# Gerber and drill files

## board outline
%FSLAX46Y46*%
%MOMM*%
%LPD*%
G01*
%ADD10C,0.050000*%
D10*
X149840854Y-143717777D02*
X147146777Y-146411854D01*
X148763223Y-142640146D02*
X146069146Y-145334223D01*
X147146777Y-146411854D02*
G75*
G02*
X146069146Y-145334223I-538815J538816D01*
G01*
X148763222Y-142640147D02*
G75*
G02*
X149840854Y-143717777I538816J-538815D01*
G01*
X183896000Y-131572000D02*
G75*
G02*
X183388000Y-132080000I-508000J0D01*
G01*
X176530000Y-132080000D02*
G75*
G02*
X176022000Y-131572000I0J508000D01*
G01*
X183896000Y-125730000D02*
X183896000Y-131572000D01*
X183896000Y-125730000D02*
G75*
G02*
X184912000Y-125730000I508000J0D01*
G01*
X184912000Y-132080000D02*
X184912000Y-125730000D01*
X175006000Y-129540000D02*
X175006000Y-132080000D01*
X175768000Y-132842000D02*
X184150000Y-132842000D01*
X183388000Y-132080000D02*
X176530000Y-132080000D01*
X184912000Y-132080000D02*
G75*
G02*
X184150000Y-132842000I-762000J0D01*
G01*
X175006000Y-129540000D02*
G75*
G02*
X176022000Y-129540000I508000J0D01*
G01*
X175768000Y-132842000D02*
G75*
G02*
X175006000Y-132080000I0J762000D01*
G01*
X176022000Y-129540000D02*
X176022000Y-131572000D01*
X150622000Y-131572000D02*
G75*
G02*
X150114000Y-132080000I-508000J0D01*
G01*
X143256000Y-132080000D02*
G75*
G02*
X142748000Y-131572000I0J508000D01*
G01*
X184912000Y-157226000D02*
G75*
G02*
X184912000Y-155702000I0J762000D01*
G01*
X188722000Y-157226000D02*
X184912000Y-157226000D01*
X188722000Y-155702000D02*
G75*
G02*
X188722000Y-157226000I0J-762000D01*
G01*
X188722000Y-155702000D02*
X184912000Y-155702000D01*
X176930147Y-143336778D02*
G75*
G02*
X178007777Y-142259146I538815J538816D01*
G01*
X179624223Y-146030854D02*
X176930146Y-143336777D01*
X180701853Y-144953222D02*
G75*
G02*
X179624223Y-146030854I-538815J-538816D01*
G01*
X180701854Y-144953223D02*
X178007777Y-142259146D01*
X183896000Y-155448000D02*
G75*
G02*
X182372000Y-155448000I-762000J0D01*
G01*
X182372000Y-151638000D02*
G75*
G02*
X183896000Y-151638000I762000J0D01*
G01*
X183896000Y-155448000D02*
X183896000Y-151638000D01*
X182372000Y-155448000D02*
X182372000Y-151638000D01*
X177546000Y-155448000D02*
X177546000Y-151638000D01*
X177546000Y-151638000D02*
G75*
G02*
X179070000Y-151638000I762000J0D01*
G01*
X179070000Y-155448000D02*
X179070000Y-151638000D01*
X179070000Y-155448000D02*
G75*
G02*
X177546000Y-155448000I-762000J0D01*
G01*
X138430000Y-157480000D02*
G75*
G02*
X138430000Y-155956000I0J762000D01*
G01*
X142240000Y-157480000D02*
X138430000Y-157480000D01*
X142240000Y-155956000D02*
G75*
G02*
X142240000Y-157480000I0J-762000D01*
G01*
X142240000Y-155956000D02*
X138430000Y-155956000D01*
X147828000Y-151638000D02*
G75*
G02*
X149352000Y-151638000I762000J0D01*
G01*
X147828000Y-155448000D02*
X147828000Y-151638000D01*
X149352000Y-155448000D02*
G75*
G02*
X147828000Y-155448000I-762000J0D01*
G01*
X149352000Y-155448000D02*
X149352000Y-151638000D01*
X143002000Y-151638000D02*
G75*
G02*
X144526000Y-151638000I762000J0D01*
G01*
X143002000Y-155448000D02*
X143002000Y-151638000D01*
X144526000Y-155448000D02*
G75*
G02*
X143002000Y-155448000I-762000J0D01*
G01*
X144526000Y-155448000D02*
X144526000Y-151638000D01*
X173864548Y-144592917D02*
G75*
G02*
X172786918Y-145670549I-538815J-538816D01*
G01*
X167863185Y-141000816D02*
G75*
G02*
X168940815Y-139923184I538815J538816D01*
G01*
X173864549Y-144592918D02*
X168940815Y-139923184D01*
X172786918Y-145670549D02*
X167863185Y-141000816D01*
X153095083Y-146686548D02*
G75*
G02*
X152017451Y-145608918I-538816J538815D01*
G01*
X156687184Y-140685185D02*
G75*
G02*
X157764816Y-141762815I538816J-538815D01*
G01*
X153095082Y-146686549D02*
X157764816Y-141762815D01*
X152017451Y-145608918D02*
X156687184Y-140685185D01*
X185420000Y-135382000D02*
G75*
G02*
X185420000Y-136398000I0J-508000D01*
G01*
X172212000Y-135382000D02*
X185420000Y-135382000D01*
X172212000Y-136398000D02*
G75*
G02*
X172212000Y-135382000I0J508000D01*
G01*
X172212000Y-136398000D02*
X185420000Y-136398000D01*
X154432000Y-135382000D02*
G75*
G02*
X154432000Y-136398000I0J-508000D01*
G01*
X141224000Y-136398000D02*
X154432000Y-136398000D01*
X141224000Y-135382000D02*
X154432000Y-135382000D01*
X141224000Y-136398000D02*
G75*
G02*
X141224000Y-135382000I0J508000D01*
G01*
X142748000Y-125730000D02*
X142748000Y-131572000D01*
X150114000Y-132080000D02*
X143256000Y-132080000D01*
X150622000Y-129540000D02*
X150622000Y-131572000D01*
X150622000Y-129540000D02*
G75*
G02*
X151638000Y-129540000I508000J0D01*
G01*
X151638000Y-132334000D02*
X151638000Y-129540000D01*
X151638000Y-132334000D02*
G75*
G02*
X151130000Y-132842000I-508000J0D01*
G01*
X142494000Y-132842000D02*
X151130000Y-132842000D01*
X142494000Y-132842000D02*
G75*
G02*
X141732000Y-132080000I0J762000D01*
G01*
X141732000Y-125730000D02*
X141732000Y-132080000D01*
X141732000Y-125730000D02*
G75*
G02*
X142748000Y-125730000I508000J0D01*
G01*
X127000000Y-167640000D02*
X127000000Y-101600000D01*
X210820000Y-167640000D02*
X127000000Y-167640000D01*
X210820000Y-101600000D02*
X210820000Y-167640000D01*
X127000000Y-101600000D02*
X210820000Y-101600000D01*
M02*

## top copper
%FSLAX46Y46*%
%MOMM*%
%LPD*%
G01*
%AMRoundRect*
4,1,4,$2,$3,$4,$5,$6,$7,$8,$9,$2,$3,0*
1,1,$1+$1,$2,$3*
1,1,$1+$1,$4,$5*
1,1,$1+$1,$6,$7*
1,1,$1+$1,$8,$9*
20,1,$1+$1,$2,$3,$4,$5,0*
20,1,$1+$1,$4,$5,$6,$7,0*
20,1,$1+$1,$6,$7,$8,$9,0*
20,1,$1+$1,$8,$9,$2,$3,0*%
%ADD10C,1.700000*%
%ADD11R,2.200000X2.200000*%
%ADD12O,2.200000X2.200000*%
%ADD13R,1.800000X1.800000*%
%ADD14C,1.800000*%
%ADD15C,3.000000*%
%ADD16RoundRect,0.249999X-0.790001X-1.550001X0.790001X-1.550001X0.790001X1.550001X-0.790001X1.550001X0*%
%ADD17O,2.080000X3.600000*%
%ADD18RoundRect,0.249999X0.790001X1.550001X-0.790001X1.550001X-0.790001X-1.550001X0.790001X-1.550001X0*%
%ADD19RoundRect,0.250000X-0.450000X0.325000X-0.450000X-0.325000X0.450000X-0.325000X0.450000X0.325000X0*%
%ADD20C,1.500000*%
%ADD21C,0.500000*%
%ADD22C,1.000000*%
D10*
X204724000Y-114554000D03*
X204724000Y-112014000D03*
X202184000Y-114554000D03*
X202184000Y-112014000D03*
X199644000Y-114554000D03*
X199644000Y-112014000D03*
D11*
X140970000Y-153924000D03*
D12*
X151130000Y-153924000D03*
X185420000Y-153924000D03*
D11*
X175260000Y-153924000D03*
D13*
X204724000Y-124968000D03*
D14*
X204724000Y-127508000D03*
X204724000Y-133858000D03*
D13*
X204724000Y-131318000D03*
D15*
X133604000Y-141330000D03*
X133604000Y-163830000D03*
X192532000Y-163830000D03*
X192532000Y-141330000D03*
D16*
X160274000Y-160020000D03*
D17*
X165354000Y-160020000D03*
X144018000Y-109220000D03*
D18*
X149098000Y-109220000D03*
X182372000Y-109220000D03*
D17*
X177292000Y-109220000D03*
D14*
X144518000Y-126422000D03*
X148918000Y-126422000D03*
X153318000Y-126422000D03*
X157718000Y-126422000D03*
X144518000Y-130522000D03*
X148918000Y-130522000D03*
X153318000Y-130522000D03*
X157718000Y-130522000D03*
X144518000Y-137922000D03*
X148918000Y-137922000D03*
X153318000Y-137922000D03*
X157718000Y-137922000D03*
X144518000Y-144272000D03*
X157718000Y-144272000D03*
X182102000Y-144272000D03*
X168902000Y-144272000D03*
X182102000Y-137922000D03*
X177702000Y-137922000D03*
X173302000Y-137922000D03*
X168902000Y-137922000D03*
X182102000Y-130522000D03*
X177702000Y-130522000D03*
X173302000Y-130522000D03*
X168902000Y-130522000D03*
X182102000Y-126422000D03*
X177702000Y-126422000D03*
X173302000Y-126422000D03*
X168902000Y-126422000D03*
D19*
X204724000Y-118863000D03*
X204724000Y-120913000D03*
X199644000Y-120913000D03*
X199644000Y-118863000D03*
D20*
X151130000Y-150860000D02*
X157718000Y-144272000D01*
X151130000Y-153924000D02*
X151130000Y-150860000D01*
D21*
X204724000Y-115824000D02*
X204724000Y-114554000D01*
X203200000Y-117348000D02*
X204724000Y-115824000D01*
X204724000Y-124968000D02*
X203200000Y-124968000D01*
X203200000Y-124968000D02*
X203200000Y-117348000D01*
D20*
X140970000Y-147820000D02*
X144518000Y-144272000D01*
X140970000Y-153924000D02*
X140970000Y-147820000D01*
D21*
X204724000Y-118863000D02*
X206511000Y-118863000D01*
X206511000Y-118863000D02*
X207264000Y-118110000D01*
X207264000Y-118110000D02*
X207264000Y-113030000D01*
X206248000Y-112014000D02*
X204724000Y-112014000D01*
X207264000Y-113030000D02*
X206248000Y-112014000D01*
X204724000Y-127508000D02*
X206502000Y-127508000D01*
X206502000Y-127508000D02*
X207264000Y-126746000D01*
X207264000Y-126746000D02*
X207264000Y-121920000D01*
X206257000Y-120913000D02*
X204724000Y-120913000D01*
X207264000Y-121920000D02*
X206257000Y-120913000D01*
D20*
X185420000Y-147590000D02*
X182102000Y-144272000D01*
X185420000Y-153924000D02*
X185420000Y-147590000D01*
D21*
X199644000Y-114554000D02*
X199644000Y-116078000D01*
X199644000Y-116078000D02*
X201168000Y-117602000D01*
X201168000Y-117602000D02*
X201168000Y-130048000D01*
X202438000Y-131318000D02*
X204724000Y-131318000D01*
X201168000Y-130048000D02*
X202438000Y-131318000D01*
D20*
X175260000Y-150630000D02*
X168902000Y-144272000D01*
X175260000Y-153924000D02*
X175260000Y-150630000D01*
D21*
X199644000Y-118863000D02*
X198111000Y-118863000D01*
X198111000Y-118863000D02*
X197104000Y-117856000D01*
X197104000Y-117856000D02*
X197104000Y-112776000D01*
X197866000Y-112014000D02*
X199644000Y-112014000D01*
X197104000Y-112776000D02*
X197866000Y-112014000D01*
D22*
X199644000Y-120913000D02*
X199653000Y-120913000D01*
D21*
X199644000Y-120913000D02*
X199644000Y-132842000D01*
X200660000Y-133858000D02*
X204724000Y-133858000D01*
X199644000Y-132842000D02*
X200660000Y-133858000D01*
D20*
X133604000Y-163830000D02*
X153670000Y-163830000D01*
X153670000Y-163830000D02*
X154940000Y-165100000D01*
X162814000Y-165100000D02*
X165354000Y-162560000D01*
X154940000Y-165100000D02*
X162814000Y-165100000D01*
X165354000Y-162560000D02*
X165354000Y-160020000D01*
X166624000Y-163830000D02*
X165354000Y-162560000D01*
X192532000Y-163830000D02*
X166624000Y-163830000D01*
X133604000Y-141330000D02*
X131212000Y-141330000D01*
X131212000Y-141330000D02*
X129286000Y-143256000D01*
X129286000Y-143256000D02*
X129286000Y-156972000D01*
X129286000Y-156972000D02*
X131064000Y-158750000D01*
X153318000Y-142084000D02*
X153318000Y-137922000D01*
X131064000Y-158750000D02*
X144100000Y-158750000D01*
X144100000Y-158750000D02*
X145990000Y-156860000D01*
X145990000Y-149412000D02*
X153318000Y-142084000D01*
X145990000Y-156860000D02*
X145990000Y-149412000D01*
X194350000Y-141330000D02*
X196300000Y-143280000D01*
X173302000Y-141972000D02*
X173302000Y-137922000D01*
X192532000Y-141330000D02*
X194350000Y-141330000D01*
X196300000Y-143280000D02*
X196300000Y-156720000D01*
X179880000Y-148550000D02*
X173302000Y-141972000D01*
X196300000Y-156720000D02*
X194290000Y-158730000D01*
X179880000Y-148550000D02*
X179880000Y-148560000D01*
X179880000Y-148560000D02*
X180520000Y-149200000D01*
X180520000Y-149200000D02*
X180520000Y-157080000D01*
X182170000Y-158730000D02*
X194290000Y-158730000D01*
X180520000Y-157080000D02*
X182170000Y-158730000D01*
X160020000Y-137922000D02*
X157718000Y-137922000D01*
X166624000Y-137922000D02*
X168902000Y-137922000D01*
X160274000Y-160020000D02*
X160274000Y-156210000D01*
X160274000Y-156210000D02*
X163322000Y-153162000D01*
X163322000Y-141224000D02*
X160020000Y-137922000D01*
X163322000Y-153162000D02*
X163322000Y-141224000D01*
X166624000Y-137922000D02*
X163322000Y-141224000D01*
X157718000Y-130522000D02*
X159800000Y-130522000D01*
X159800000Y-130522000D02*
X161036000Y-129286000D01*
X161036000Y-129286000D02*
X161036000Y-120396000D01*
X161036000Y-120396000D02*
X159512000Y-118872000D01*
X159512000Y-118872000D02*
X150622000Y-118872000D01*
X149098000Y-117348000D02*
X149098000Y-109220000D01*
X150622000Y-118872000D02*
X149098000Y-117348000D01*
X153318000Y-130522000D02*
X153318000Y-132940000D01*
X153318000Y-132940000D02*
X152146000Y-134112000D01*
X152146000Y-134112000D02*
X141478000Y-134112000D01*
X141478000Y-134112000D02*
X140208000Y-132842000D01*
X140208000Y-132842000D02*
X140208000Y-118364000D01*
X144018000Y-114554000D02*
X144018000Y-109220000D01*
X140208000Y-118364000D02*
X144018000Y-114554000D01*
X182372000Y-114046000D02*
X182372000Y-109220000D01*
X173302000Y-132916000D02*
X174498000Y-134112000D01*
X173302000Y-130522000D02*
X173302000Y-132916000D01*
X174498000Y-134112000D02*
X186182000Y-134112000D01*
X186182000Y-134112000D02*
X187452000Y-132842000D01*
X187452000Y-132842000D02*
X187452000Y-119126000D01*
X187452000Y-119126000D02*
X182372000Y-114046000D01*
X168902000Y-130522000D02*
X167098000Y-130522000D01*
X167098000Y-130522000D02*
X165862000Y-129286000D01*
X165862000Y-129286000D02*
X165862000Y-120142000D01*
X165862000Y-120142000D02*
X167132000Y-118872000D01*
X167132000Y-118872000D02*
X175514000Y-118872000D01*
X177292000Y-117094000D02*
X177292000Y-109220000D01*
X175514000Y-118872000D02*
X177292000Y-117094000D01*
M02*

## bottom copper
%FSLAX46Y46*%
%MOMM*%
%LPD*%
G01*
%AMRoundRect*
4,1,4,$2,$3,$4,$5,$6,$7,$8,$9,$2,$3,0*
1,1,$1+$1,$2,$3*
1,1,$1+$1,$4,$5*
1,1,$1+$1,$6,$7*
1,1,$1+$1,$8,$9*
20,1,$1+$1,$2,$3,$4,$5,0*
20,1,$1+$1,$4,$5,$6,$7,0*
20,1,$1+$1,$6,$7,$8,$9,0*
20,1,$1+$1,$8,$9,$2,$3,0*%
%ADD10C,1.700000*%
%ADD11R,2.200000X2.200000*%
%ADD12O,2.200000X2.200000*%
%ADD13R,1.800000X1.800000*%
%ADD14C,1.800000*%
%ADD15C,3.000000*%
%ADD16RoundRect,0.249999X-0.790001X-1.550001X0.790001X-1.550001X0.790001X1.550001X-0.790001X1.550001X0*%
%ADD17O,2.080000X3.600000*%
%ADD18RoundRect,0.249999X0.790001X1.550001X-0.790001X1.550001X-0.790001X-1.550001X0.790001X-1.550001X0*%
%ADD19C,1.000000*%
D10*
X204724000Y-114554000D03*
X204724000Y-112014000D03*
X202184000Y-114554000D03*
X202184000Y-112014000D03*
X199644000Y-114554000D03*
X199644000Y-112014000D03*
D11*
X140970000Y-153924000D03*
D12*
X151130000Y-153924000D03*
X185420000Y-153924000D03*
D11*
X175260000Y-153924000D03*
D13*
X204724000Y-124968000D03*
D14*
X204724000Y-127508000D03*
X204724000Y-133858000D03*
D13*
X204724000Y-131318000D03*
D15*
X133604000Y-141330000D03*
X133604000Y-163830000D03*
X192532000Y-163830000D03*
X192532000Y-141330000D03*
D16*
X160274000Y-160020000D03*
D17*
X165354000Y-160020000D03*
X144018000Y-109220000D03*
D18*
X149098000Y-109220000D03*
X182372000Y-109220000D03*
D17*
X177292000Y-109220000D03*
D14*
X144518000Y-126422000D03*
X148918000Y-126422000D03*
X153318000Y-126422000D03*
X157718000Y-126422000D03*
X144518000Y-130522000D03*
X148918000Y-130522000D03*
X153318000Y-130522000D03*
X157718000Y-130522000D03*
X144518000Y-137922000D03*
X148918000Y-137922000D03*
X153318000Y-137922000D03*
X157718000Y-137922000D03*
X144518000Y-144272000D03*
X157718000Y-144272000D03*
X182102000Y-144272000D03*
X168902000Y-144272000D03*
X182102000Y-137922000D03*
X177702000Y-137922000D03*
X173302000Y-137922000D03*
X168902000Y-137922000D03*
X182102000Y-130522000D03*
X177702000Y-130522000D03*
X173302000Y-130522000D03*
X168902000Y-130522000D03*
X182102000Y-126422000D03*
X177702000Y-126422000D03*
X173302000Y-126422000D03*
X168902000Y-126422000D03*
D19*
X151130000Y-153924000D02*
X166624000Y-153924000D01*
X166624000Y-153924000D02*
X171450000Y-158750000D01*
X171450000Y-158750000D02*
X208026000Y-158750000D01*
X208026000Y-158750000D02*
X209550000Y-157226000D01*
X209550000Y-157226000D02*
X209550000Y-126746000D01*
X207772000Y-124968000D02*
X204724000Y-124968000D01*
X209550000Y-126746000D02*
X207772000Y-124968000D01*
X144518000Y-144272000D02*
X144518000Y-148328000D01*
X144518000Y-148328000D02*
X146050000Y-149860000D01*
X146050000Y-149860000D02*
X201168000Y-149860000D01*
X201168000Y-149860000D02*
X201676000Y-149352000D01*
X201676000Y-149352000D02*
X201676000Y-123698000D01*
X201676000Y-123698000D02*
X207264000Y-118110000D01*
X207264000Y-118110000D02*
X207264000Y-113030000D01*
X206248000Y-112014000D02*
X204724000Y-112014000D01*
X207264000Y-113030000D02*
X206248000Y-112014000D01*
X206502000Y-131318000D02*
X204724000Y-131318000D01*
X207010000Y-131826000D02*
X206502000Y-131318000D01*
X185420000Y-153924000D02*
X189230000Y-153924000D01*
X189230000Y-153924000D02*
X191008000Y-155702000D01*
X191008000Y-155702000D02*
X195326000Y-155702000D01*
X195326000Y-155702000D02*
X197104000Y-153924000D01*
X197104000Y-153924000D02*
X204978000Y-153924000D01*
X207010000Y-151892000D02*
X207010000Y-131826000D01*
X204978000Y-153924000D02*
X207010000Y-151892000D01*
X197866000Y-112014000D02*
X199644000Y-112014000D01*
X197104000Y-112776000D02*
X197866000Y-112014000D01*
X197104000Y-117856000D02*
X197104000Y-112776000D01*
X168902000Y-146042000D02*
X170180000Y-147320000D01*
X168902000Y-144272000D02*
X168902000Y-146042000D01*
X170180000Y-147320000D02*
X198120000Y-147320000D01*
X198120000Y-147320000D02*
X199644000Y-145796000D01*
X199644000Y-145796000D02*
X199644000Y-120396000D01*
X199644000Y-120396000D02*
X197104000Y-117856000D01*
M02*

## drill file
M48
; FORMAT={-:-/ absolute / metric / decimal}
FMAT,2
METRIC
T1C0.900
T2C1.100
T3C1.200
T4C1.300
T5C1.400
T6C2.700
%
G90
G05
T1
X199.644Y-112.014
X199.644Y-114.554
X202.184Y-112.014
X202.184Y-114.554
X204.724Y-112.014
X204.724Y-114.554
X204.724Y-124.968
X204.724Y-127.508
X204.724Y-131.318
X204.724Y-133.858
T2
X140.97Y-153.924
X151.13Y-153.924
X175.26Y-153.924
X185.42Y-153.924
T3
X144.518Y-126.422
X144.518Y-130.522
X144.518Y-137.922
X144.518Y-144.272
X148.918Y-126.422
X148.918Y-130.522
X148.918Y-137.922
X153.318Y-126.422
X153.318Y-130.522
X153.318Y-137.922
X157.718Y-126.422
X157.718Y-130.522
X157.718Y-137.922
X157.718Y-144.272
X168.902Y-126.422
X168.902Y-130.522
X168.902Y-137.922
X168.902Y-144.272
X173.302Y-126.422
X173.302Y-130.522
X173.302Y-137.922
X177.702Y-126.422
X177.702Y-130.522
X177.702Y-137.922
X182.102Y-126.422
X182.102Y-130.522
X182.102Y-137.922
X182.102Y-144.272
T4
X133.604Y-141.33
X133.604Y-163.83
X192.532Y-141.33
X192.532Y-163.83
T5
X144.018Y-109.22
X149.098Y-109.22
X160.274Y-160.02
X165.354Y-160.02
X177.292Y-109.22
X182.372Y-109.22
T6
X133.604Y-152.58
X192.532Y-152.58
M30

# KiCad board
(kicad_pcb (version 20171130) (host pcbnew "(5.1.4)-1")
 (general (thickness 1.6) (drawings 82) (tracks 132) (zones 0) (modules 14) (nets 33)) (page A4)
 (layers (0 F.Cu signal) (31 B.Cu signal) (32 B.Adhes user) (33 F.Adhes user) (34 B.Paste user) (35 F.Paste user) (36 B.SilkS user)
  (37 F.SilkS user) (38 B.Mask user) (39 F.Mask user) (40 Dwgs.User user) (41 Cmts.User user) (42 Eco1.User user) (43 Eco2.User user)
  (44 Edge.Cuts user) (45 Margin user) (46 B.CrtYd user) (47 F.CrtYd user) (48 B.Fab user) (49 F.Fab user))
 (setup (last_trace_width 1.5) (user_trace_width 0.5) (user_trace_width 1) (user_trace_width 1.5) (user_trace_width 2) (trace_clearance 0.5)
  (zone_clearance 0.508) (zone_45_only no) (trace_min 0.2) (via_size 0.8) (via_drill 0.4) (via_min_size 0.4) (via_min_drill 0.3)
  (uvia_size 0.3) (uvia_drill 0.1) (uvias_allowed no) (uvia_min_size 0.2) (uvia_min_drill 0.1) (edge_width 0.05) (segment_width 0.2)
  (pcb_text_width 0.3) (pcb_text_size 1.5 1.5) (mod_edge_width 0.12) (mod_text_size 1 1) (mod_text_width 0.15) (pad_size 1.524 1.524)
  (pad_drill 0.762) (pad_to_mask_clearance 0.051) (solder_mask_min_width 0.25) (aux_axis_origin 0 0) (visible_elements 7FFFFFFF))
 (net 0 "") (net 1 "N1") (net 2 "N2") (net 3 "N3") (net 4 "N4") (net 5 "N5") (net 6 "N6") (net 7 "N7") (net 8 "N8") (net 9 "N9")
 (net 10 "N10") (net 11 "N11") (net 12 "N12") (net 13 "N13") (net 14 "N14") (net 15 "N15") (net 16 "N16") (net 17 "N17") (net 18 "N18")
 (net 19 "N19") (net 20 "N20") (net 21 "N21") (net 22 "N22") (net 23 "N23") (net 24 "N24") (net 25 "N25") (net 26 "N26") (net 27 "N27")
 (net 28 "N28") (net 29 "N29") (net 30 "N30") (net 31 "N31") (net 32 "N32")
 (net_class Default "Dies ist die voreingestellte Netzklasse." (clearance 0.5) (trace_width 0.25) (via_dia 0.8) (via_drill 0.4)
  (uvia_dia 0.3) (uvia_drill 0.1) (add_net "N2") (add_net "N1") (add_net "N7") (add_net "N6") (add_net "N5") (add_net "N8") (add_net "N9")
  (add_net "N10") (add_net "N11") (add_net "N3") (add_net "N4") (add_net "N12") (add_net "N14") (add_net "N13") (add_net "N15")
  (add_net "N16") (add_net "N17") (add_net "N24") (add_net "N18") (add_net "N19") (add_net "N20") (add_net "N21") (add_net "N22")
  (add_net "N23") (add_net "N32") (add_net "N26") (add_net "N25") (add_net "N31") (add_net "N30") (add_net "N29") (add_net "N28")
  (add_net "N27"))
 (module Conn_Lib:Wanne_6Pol (layer F.Cu) (at 202.184 109.474 270)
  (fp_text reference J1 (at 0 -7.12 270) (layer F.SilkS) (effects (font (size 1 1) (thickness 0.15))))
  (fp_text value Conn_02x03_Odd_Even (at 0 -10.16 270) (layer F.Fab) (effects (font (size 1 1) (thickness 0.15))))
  (pad 1 thru_hole circle (at 5.08 -2.54 270) (size 1.7 1.7) (drill 0.9) (layers *.Cu *.Mask) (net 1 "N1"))
  (pad 2 thru_hole circle (at 2.54 -2.54 270) (size 1.7 1.7) (drill 0.9) (layers *.Cu *.Mask) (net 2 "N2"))
  (pad 3 thru_hole circle (at 5.08 0 270) (size 1.7 1.7) (drill 0.9) (layers *.Cu *.Mask) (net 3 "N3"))
  (pad 4 thru_hole circle (at 2.54 0 270) (size 1.7 1.7) (drill 0.9) (layers *.Cu *.Mask) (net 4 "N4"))
  (pad 5 thru_hole circle (at 5.08 2.54 270) (size 1.7 1.7) (drill 0.9) (layers *.Cu *.Mask) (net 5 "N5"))
  (pad 6 thru_hole circle (at 2.54 2.54 270) (size 1.7 1.7) (drill 0.9) (layers *.Cu *.Mask) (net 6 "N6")))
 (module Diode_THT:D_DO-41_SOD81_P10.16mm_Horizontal (layer F.Cu) (at 140.97 153.924)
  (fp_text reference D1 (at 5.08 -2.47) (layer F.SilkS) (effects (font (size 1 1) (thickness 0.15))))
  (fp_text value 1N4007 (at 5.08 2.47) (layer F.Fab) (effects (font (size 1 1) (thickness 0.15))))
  (pad 1 thru_hole rect (at 0 0) (size 2.2 2.2) (drill 1.1) (layers *.Cu *.Mask) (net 2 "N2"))
  (pad 2 thru_hole oval (at 10.16 0) (size 2.2 2.2) (drill 1.1) (layers *.Cu *.Mask) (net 1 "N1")))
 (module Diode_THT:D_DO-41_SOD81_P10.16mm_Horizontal (layer F.Cu) (at 175.26 153.924)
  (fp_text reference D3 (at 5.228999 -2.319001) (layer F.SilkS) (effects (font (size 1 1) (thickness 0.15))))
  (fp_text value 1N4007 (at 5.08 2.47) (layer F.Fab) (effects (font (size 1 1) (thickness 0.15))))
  (pad 2 thru_hole oval (at 10.16 0) (size 2.2 2.2) (drill 1.1) (layers *.Cu *.Mask) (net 5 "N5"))
  (pad 1 thru_hole rect (at 0 0) (size 2.2 2.2) (drill 1.1) (layers *.Cu *.Mask) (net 6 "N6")))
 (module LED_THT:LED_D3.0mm (layer F.Cu) (at 204.724 124.968 270)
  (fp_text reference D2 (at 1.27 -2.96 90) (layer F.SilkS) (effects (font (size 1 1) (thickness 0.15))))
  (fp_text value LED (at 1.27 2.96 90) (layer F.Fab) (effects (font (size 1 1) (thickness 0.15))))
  (pad 1 thru_hole rect (at 0 0 270) (size 1.8 1.8) (drill 0.9) (layers *.Cu *.Mask) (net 1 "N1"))
  (pad 2 thru_hole circle (at 2.54 0 270) (size 1.8 1.8) (drill 0.9) (layers *.Cu *.Mask) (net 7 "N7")))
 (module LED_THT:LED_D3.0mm (layer F.Cu) (at 204.724 131.318 270)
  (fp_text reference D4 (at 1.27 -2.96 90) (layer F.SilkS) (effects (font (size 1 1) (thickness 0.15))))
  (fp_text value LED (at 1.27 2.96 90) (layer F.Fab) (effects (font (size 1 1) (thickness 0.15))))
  (pad 2 thru_hole circle (at 2.54 0 270) (size 1.8 1.8) (drill 0.9) (layers *.Cu *.Mask) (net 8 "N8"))
  (pad 1 thru_hole rect (at 0 0 270) (size 1.8 1.8) (drill 0.9) (layers *.Cu *.Mask) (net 5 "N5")))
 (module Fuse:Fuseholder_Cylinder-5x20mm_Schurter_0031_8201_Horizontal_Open (layer F.Cu) (at 133.604 141.33 270)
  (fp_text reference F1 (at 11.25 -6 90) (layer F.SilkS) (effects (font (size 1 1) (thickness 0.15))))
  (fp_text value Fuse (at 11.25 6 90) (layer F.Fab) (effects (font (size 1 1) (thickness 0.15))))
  (pad 1 thru_hole circle (at 0 0 270) (size 3 3) (drill 1.3) (layers *.Cu *.Mask) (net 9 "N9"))
  (pad 2 thru_hole circle (at 22.5 0 270) (size 3 3) (drill 1.3) (layers *.Cu *.Mask) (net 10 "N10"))
  (pad "" np_thru_hole circle (at 11.25 0 270) (size 2.7 2.7) (drill 2.7) (layers *.Cu *.Mask)))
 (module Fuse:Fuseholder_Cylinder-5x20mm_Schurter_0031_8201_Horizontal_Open (layer F.Cu) (at 192.532 141.33 270)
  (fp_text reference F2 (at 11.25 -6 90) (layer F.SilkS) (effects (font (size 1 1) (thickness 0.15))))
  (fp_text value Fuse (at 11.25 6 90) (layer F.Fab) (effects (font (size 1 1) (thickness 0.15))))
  (pad "" np_thru_hole circle (at 11.25 0 270) (size 2.7 2.7) (drill 2.7) (layers *.Cu *.Mask))
  (pad 2 thru_hole circle (at 22.5 0 270) (size 3 3) (drill 1.3) (layers *.Cu *.Mask) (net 10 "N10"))
  (pad 1 thru_hole circle (at 0 0 270) (size 3 3) (drill 1.3) (layers *.Cu *.Mask) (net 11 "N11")))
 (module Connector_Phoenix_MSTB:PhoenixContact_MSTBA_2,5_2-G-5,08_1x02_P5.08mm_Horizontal (layer F.Cu) (at 160.274 160.02)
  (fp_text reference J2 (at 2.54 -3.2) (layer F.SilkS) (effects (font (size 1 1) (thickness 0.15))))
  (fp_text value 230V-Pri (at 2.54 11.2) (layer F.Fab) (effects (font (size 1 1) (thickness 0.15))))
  (pad 1 thru_hole roundrect (at 0 0) (size 2.08 3.6) (drill 1.4) (layers *.Cu *.Mask) (roundrect_rratio 0.120192) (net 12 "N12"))
  (pad 2 thru_hole oval (at 5.08 0) (size 2.08 3.6) (drill 1.4) (layers *.Cu *.Mask) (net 10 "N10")))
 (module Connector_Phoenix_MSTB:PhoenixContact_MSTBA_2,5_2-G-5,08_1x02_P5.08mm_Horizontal (layer F.Cu) (at 149.098 109.22 180)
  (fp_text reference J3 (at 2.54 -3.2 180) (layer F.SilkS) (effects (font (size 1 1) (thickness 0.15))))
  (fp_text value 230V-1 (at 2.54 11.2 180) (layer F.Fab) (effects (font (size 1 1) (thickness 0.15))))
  (pad 2 thru_hole oval (at 5.08 0 180) (size 2.08 3.6) (drill 1.4) (layers *.Cu *.Mask) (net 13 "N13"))
  (pad 1 thru_hole roundrect (at 0 0 180) (size 2.08 3.6) (drill 1.4) (layers *.Cu *.Mask) (roundrect_rratio 0.120192) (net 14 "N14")))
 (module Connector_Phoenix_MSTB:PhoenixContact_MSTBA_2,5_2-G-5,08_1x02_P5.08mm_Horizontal (layer F.Cu) (at 182.372 109.22 180)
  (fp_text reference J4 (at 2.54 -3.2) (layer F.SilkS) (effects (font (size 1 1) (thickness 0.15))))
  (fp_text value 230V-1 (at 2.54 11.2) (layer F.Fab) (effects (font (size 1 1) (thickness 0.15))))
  (pad 1 thru_hole roundrect (at 0 0 180) (size 2.08 3.6) (drill 1.4) (layers *.Cu *.Mask) (roundrect_rratio 0.120192) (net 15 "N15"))
  (pad 2 thru_hole oval (at 5.08 0 180) (size 2.08 3.6) (drill 1.4) (layers *.Cu *.Mask) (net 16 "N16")))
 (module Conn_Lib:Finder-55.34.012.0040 (layer F.Cu) (at 151.638 134.112)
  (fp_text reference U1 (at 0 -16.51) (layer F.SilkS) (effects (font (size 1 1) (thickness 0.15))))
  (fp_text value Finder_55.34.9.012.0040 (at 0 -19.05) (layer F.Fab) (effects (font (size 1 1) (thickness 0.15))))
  (pad 1 thru_hole circle (at -7.12 -7.69) (size 1.8 1.8) (drill 1.2) (layers *.Cu *.Mask) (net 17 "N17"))
  (pad 2 thru_hole circle (at -2.72 -7.69) (size 1.8 1.8) (drill 1.2) (layers *.Cu *.Mask) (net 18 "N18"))
  (pad 3 thru_hole circle (at 1.68 -7.69) (size 1.8 1.8) (drill 1.2) (layers *.Cu *.Mask) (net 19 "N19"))
  (pad 4 thru_hole circle (at 6.08 -7.69) (size 1.8 1.8) (drill 1.2) (layers *.Cu *.Mask) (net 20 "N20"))
  (pad 5 thru_hole circle (at -7.12 -3.59) (size 1.8 1.8) (drill 1.2) (layers *.Cu *.Mask) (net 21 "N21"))
  (pad 6 thru_hole circle (at -2.72 -3.59) (size 1.8 1.8) (drill 1.2) (layers *.Cu *.Mask) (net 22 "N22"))
  (pad 7 thru_hole circle (at 1.68 -3.59) (size 1.8 1.8) (drill 1.2) (layers *.Cu *.Mask) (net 13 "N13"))
  (pad 8 thru_hole circle (at 6.08 -3.59) (size 1.8 1.8) (drill 1.2) (layers *.Cu *.Mask) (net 14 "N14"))
  (pad 9 thru_hole circle (at -7.12 3.81) (size 1.8 1.8) (drill 1.2) (layers *.Cu *.Mask) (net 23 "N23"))
  (pad 10 thru_hole circle (at -2.72 3.81) (size 1.8 1.8) (drill 1.2) (layers *.Cu *.Mask) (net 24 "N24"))
  (pad 11 thru_hole circle (at 1.68 3.81) (size 1.8 1.8) (drill 1.2) (layers *.Cu *.Mask) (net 9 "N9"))
  (pad 12 thru_hole circle (at 6.08 3.81) (size 1.8 1.8) (drill 1.2) (layers *.Cu *.Mask) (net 12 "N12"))
  (pad 13 thru_hole circle (at -7.12 10.16) (size 1.8 1.8) (drill 1.2) (layers *.Cu *.Mask) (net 2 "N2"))
  (pad 14 thru_hole circle (at 6.08 10.16) (size 1.8 1.8) (drill 1.2) (layers *.Cu *.Mask) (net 1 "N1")))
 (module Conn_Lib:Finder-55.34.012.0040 (layer F.Cu) (at 176.022 134.112)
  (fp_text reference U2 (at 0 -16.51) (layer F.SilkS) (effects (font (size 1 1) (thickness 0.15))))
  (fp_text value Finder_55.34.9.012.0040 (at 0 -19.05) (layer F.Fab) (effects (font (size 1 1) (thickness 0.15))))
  (pad 14 thru_hole circle (at 6.08 10.16) (size 1.8 1.8) (drill 1.2) (layers *.Cu *.Mask) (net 5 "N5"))
  (pad 13 thru_hole circle (at -7.12 10.16) (size 1.8 1.8) (drill 1.2) (layers *.Cu *.Mask) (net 6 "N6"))
  (pad 12 thru_hole circle (at 6.08 3.81) (size 1.8 1.8) (drill 1.2) (layers *.Cu *.Mask) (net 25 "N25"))
  (pad 11 thru_hole circle (at 1.68 3.81) (size 1.8 1.8) (drill 1.2) (layers *.Cu *.Mask) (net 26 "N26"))
  (pad 10 thru_hole circle (at -2.72 3.81) (size 1.8 1.8) (drill 1.2) (layers *.Cu *.Mask) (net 11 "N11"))
  (pad 9 thru_hole circle (at -7.12 3.81) (size 1.8 1.8) (drill 1.2) (layers *.Cu *.Mask) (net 12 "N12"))
  (pad 8 thru_hole circle (at 6.08 -3.59) (size 1.8 1.8) (drill 1.2) (layers *.Cu *.Mask) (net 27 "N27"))
  (pad 7 thru_hole circle (at 1.68 -3.59) (size 1.8 1.8) (drill 1.2) (layers *.Cu *.Mask) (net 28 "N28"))
  (pad 6 thru_hole circle (at -2.72 -3.59) (size 1.8 1.8) (drill 1.2) (layers *.Cu *.Mask) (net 15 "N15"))
  (pad 5 thru_hole circle (at -7.12 -3.59) (size 1.8 1.8) (drill 1.2) (layers *.Cu *.Mask) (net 16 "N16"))
  (pad 4 thru_hole circle (at 6.08 -7.69) (size 1.8 1.8) (drill 1.2) (layers *.Cu *.Mask) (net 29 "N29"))
  (pad 3 thru_hole circle (at 1.68 -7.69) (size 1.8 1.8) (drill 1.2) (layers *.Cu *.Mask) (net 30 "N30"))
  (pad 2 thru_hole circle (at -2.72 -7.69) (size 1.8 1.8) (drill 1.2) (layers *.Cu *.Mask) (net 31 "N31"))
  (pad 1 thru_hole circle (at -7.12 -7.69) (size 1.8 1.8) (drill 1.2) (layers *.Cu *.Mask) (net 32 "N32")))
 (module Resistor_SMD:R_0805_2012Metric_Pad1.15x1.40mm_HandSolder (layer F.Cu) (at 204.724 119.888 270)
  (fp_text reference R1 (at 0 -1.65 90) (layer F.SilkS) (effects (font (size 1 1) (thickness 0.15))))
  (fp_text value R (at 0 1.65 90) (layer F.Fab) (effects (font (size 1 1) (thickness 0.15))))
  (pad 1 smd roundrect (at -1.025 0 270) (size 1.15 1.4) (layers F.Cu F.Paste F.Mask) (roundrect_rratio 0.217391) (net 2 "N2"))
  (pad 2 smd roundrect (at 1.025 0 270) (size 1.15 1.4) (layers F.Cu F.Paste F.Mask) (roundrect_rratio 0.217391) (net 7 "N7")))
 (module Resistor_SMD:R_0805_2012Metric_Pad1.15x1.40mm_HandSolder (layer F.Cu) (at 199.644 119.888 270)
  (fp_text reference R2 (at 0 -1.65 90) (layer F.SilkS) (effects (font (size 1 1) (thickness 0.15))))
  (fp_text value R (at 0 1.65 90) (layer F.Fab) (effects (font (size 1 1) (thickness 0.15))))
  (pad 2 smd roundrect (at 1.025 0 270) (size 1.15 1.4) (layers F.Cu F.Paste F.Mask) (roundrect_rratio 0.217391) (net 8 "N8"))
  (pad 1 smd roundrect (at -1.025 0 270) (size 1.15 1.4) (layers F.Cu F.Paste F.Mask) (roundrect_rratio 0.217391) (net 6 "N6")))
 (gr_line (start 149.840854 143.717777) (end 147.146777 146.411854) (layer Edge.Cuts) (width 0.05))
 (gr_line (start 148.763223 142.640146) (end 146.069146 145.334223) (layer Edge.Cuts) (width 0.05))
 (gr_arc (start 146.607962 145.873038) (end 146.069146 145.334223) (angle -179.9998937) (layer Edge.Cuts) (width 0.05))
 (gr_arc (start 149.302038 143.178962) (end 149.840854 143.717777) (angle -180) (layer Edge.Cuts) (width 0.05))
 (gr_arc (start 183.388 131.572) (end 183.388 132.08) (angle -90) (layer Edge.Cuts) (width 0.05))
 (gr_arc (start 176.53 131.572) (end 176.022 131.572) (angle -90) (layer Edge.Cuts) (width 0.05))
 (gr_line (start 183.896 125.73) (end 183.896 131.572) (layer Edge.Cuts) (width 0.05))
 (gr_arc (start 184.404 125.73) (end 184.912 125.73) (angle -180) (layer Edge.Cuts) (width 0.05))
 (gr_line (start 184.912 132.08) (end 184.912 125.73) (layer Edge.Cuts) (width 0.05))
 (gr_line (start 175.006 129.54) (end 175.006 132.08) (layer Edge.Cuts) (width 0.05))
 (gr_line (start 175.768 132.842) (end 184.15 132.842) (layer Edge.Cuts) (width 0.05))
 (gr_line (start 183.388 132.08) (end 176.53 132.08) (layer Edge.Cuts) (width 0.05))
 (gr_arc (start 184.15 132.08) (end 184.15 132.842) (angle -90) (layer Edge.Cuts) (width 0.05))
 (gr_arc (start 175.514 129.54) (end 176.022 129.54) (angle -180) (layer Edge.Cuts) (width 0.05))
 (gr_arc (start 175.768 132.08) (end 175.006 132.08) (angle -90) (layer Edge.Cuts) (width 0.05))
 (gr_line (start 176.022 129.54) (end 176.022 131.572) (layer Edge.Cuts) (width 0.05))
 (gr_arc (start 150.114 131.572) (end 150.114 132.08) (angle -90) (layer Edge.Cuts) (width 0.05))
 (gr_arc (start 143.256 131.572) (end 142.748 131.572) (angle -90) (layer Edge.Cuts) (width 0.05))
 (gr_arc (start 184.912 156.464) (end 184.912 155.702) (angle -180) (layer Edge.Cuts) (width 0.05))
 (gr_line (start 188.722 157.226) (end 184.912 157.226) (layer Edge.Cuts) (width 0.05))
 (gr_arc (start 188.722 156.464) (end 188.722 157.226) (angle -180) (layer Edge.Cuts) (width 0.05))
 (gr_line (start 188.722 155.702) (end 184.912 155.702) (layer Edge.Cuts) (width 0.05))
 (gr_arc (start 177.468962 142.797962) (end 178.007777 142.259146) (angle -180) (layer Edge.Cuts) (width 0.05))
 (gr_line (start 179.624223 146.030854) (end 176.930146 143.336777) (layer Edge.Cuts) (width 0.05))
 (gr_arc (start 180.163038 145.492038) (end 179.624223 146.030854) (angle -180) (layer Edge.Cuts) (width 0.05))
 (gr_line (start 180.701854 144.953223) (end 178.007777 142.259146) (layer Edge.Cuts) (width 0.05))
 (gr_arc (start 183.134 155.448) (end 182.372 155.448) (angle -180) (layer Edge.Cuts) (width 0.05))
 (gr_arc (start 183.134 151.638) (end 183.896 151.638) (angle -180) (layer Edge.Cuts) (width 0.05))
 (gr_line (start 183.896 155.448) (end 183.896 151.638) (layer Edge.Cuts) (width 0.05))
 (gr_line (start 182.372 155.448) (end 182.372 151.638) (layer Edge.Cuts) (width 0.05))
 (gr_line (start 177.546 155.448) (end 177.546 151.638) (layer Edge.Cuts) (width 0.05))
 (gr_arc (start 178.308 151.638) (end 179.07 151.638) (angle -180) (layer Edge.Cuts) (width 0.05))
 (gr_line (start 179.07 155.448) (end 179.07 151.638) (layer Edge.Cuts) (width 0.05))
 (gr_arc (start 178.308 155.448) (end 177.546 155.448) (angle -180) (layer Edge.Cuts) (width 0.05))
 (gr_arc (start 138.43 156.718) (end 138.43 155.956) (angle -180) (layer Edge.Cuts) (width 0.05))
 (gr_line (start 142.24 157.48) (end 138.43 157.48) (layer Edge.Cuts) (width 0.05))
 (gr_arc (start 142.24 156.718) (end 142.24 157.48) (angle -180) (layer Edge.Cuts) (width 0.05))
 (gr_line (start 142.24 155.956) (end 138.43 155.956) (layer Edge.Cuts) (width 0.05))
 (gr_arc (start 148.59 151.638) (end 149.352 151.638) (angle -180) (layer Edge.Cuts) (width 0.05))
 (gr_line (start 147.828 155.448) (end 147.828 151.638) (layer Edge.Cuts) (width 0.05))
 (gr_arc (start 148.59 155.448) (end 147.828 155.448) (angle -180) (layer Edge.Cuts) (width 0.05))
 (gr_line (start 149.352 155.448) (end 149.352 151.638) (layer Edge.Cuts) (width 0.05))
 (gr_arc (start 143.764 151.638) (end 144.526 151.638) (angle -180) (layer Edge.Cuts) (width 0.05))
 (gr_line (start 143.002 155.448) (end 143.002 151.638) (layer Edge.Cuts) (width 0.05))
 (gr_arc (start 143.764 155.448) (end 143.002 155.448) (angle -180) (layer Edge.Cuts) (width 0.05))
 (gr_line (start 144.526 155.448) (end 144.526 151.638) (layer Edge.Cuts) (width 0.05))
 (gr_arc (start 173.325733 145.131733) (end 172.786918 145.670549) (angle -180) (layer Edge.Cuts) (width 0.05))
 (gr_arc (start 168.402 140.462) (end 168.940815 139.923184) (angle -180) (layer Edge.Cuts) (width 0.05))
 (gr_line (start 173.864549 144.592918) (end 168.940815 139.923184) (layer Edge.Cuts) (width 0.05))
 (gr_line (start 172.786918 145.670549) (end 167.863185 141.000816) (layer Edge.Cuts) (width 0.05))
 (gr_arc (start 152.556267 146.147733) (end 152.017451 145.608918) (angle -180) (layer Edge.Cuts) (width 0.05))
 (gr_arc (start 157.226 141.224) (end 157.764816 141.762815) (angle -180) (layer Edge.Cuts) (width 0.05))
 (gr_line (start 153.095082 146.686549) (end 157.764816 141.762815) (layer Edge.Cuts) (width 0.05))
 (gr_line (start 152.017451 145.608918) (end 156.687184 140.685185) (layer Edge.Cuts) (width 0.05))
 (gr_arc (start 185.42 135.89) (end 185.42 136.398) (angle -180) (layer Edge.Cuts) (width 0.05))
 (gr_line (start 172.212 135.382) (end 185.42 135.382) (layer Edge.Cuts) (width 0.05))
 (gr_arc (start 172.212 135.89) (end 172.212 135.382) (angle -180) (layer Edge.Cuts) (width 0.05))
 (gr_line (start 172.212 136.398) (end 185.42 136.398) (layer Edge.Cuts) (width 0.05))
 (gr_arc (start 154.432 135.89) (end 154.432 136.398) (angle -180) (layer Edge.Cuts) (width 0.05))
 (gr_line (start 141.224 136.398) (end 154.432 136.398) (layer Edge.Cuts) (width 0.05))
 (gr_line (start 141.224 135.382) (end 154.432 135.382) (layer Edge.Cuts) (width 0.05))
 (gr_arc (start 141.224 135.89) (end 141.224 135.382) (angle -180) (layer Edge.Cuts) (width 0.05))
 (gr_line (start 142.748 125.73) (end 142.748 131.572) (layer Edge.Cuts) (width 0.05))
 (gr_line (start 150.114 132.08) (end 143.256 132.08) (layer Edge.Cuts) (width 0.05))
 (gr_line (start 150.622 129.54) (end 150.622 131.572) (layer Edge.Cuts) (width 0.05))
 (gr_arc (start 151.13 129.54) (end 151.638 129.54) (angle -180) (layer Edge.Cuts) (width 0.05))
 (gr_line (start 151.638 132.334) (end 151.638 129.54) (layer Edge.Cuts) (width 0.05))
 (gr_arc (start 151.13 132.334) (end 151.13 132.842) (angle -90) (layer Edge.Cuts) (width 0.05))
 (gr_line (start 142.494 132.842) (end 151.13 132.842) (layer Edge.Cuts) (width 0.05))
 (gr_arc (start 142.494 132.08) (end 141.732 132.08) (angle -90) (layer Edge.Cuts) (width 0.05))
 (gr_line (start 141.732 125.73) (end 141.732 132.08) (layer Edge.Cuts) (width 0.05))
 (gr_arc (start 142.24 125.73) (end 142.748 125.73) (angle -180) (layer Edge.Cuts) (width 0.05))
 (gr_line (start 127 167.64) (end 127 101.6) (layer Edge.Cuts) (width 0.05))
 (gr_line (start 210.82 167.64) (end 127 167.64) (layer Edge.Cuts) (width 0.05))
 (gr_line (start 210.82 101.6) (end 210.82 167.64) (layer Edge.Cuts) (width 0.05))
 (gr_line (start 127 101.6) (end 210.82 101.6) (layer Edge.Cuts) (width 0.05))
 (segment (start 151.13 150.86) (end 157.718 144.272) (width 1.5) (layer F.Cu) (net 1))
 (segment (start 151.13 153.924) (end 151.13 150.86) (width 1.5) (layer F.Cu) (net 1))
 (segment (start 151.13 153.924) (end 166.624 153.924) (width 1) (layer B.Cu) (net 1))
 (segment (start 166.624 153.924) (end 171.45 158.75) (width 1) (layer B.Cu) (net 1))
 (segment (start 171.45 158.75) (end 208.026 158.75) (width 1) (layer B.Cu) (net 1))
 (segment (start 208.026 158.75) (end 209.55 157.226) (width 1) (layer B.Cu) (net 1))
 (segment (start 209.55 157.226) (end 209.55 126.746) (width 1) (layer B.Cu) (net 1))
 (segment (start 207.772 124.968) (end 204.724 124.968) (width 1) (layer B.Cu) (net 1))
 (segment (start 209.55 126.746) (end 207.772 124.968) (width 1) (layer B.Cu) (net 1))
 (segment (start 204.724 115.824) (end 204.724 114.554) (width 0.5) (layer F.Cu) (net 1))
 (segment (start 203.2 117.348) (end 204.724 115.824) (width 0.5) (layer F.Cu) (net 1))
 (segment (start 204.724 124.968) (end 203.2 124.968) (width 0.5) (layer F.Cu) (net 1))
 (segment (start 203.2 124.968) (end 203.2 117.348) (width 0.5) (layer F.Cu) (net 1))
 (segment (start 140.97 147.82) (end 144.518 144.272) (width 1.5) (layer F.Cu) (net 2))
 (segment (start 140.97 153.924) (end 140.97 147.82) (width 1.5) (layer F.Cu) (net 2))
 (segment (start 144.518 144.272) (end 144.518 148.328) (width 1) (layer B.Cu) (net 2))
 (segment (start 144.518 148.328) (end 146.05 149.86) (width 1) (layer B.Cu) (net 2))
 (segment (start 146.05 149.86) (end 201.168 149.86) (width 1) (layer B.Cu) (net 2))
 (segment (start 201.168 149.86) (end 201.676 149.352) (width 1) (layer B.Cu) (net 2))
 (segment (start 201.676 149.352) (end 201.676 123.698) (width 1) (layer B.Cu) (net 2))
 (segment (start 201.676 123.698) (end 207.264 118.11) (width 1) (layer B.Cu) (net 2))
 (segment (start 207.264 118.11) (end 207.264 113.03) (width 1) (layer B.Cu) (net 2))
 (segment (start 206.248 112.014) (end 204.724 112.014) (width 1) (layer B.Cu) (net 2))
 (segment (start 207.264 113.03) (end 206.248 112.014) (width 1) (layer B.Cu) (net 2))
 (segment (start 204.724 118.863) (end 206.511 118.863) (width 0.5) (layer F.Cu) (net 2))
 (segment (start 206.511 118.863) (end 207.264 118.11) (width 0.5) (layer F.Cu) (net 2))
 (segment (start 207.264 118.11) (end 207.264 113.03) (width 0.5) (layer F.Cu) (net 2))
 (segment (start 206.248 112.014) (end 204.724 112.014) (width 0.5) (layer F.Cu) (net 2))
 (segment (start 207.264 113.03) (end 206.248 112.014) (width 0.5) (layer F.Cu) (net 2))
 (segment (start 204.724 127.508) (end 206.502 127.508) (width 0.5) (layer F.Cu) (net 7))
 (segment (start 206.502 127.508) (end 207.264 126.746) (width 0.5) (layer F.Cu) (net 7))
 (segment (start 207.264 126.746) (end 207.264 121.92) (width 0.5) (layer F.Cu) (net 7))
 (segment (start 206.257 120.913) (end 204.724 120.913) (width 0.5) (layer F.Cu) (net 7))
 (segment (start 207.264 121.92) (end 206.257 120.913) (width 0.5) (layer F.Cu) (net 7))
 (segment (start 185.42 147.59) (end 182.102 144.272) (width 1.5) (layer F.Cu) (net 5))
 (segment (start 185.42 153.924) (end 185.42 147.59) (width 1.5) (layer F.Cu) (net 5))
 (segment (start 206.502 131.318) (end 204.724 131.318) (width 1) (layer B.Cu) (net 5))
 (segment (start 207.01 131.826) (end 206.502 131.318) (width 1) (layer B.Cu) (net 5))
 (segment (start 199.644 114.554) (end 199.644 116.078) (width 0.5) (layer F.Cu) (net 5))
 (segment (start 199.644 116.078) (end 201.168 117.602) (width 0.5) (layer F.Cu) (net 5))
 (segment (start 201.168 117.602) (end 201.168 130.048) (width 0.5) (layer F.Cu) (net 5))
 (segment (start 202.438 131.318) (end 204.724 131.318) (width 0.5) (layer F.Cu) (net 5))
 (segment (start 201.168 130.048) (end 202.438 131.318) (width 0.5) (layer F.Cu) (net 5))
 (segment (start 185.42 153.924) (end 189.23 153.924) (width 1) (layer B.Cu) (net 5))
 (segment (start 189.23 153.924) (end 191.008 155.702) (width 1) (layer B.Cu) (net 5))
 (segment (start 191.008 155.702) (end 195.326 155.702) (width 1) (layer B.Cu) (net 5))
 (segment (start 195.326 155.702) (end 197.104 153.924) (width 1) (layer B.Cu) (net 5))
 (segment (start 197.104 153.924) (end 204.978 153.924) (width 1) (layer B.Cu) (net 5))
 (segment (start 207.01 151.892) (end 207.01 131.826) (width 1) (layer B.Cu) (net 5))
 (segment (start 204.978 153.924) (end 207.01 151.892) (width 1) (layer B.Cu) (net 5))
 (segment (start 175.26 150.63) (end 168.902 144.272) (width 1.5) (layer F.Cu) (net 6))
 (segment (start 175.26 153.924) (end 175.26 150.63) (width 1.5) (layer F.Cu) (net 6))
 (segment (start 197.866 112.014) (end 199.644 112.014) (width 1) (layer B.Cu) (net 6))
 (segment (start 197.104 112.776) (end 197.866 112.014) (width 1) (layer B.Cu) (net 6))
 (segment (start 197.104 117.856) (end 197.104 112.776) (width 1) (layer B.Cu) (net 6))
 (segment (start 168.902 146.042) (end 170.18 147.32) (width 1) (layer B.Cu) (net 6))
 (segment (start 168.902 144.272) (end 168.902 146.042) (width 1) (layer B.Cu) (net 6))
 (segment (start 170.18 147.32) (end 198.12 147.32) (width 1) (layer B.Cu) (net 6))
 (segment (start 198.12 147.32) (end 199.644 145.796) (width 1) (layer B.Cu) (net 6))
 (segment (start 199.644 145.796) (end 199.644 120.396) (width 1) (layer B.Cu) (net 6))
 (segment (start 199.644 120.396) (end 197.104 117.856) (width 1) (layer B.Cu) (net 6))
 (segment (start 199.644 118.863) (end 198.111 118.863) (width 0.5) (layer F.Cu) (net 6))
 (segment (start 198.111 118.863) (end 197.104 117.856) (width 0.5) (layer F.Cu) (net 6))
 (segment (start 197.104 117.856) (end 197.104 112.776) (width 0.5) (layer F.Cu) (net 6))
 (segment (start 197.866 112.014) (end 199.644 112.014) (width 0.5) (layer F.Cu) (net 6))
 (segment (start 197.104 112.776) (end 197.866 112.014) (width 0.5) (layer F.Cu) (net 6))
 (segment (start 199.644 120.913) (end 199.653 120.913) (width 1) (layer F.Cu) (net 8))
 (segment (start 199.644 120.913) (end 199.644 132.842) (width 0.5) (layer F.Cu) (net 8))
 (segment (start 200.66 133.858) (end 204.724 133.858) (width 0.5) (layer F.Cu) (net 8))
 (segment (start 199.644 132.842) (end 200.66 133.858) (width 0.5) (layer F.Cu) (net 8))
 (segment (start 133.604 163.83) (end 153.67 163.83) (width 1.5) (layer F.Cu) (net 10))
 (segment (start 153.67 163.83) (end 154.94 165.1) (width 1.5) (layer F.Cu) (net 10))
 (segment (start 162.814 165.1) (end 165.354 162.56) (width 1.5) (layer F.Cu) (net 10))
 (segment (start 154.94 165.1) (end 162.814 165.1) (width 1.5) (layer F.Cu) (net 10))
 (segment (start 165.354 162.56) (end 165.354 160.02) (width 1.5) (layer F.Cu) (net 10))
 (segment (start 166.624 163.83) (end 165.354 162.56) (width 1.5) (layer F.Cu) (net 10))
 (segment (start 192.532 163.83) (end 166.624 163.83) (width 1.5) (layer F.Cu) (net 10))
 (segment (start 133.604 141.33) (end 131.212 141.33) (width 1.5) (layer F.Cu) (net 9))
 (segment (start 131.212 141.33) (end 129.286 143.256) (width 1.5) (layer F.Cu) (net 9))
 (segment (start 129.286 143.256) (end 129.286 156.972) (width 1.5) (layer F.Cu) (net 9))
 (segment (start 129.286 156.972) (end 131.064 158.75) (width 1.5) (layer F.Cu) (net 9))
 (segment (start 153.318 142.084) (end 153.318 137.922) (width 1.5) (layer F.Cu) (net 9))
 (segment (start 131.064 158.75) (end 144.1 158.75) (width 1.5) (layer F.Cu) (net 9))
 (segment (start 144.1 158.75) (end 145.99 156.86) (width 1.5) (layer F.Cu) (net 9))
 (segment (start 145.99 149.412) (end 153.318 142.084) (width 1.5) (layer F.Cu) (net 9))
 (segment (start 145.99 156.86) (end 145.99 149.412) (width 1.5) (layer F.Cu) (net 9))
 (segment (start 194.35 141.33) (end 196.3 143.28) (width 1.5) (layer F.Cu) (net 11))
 (segment (start 173.302 141.972) (end 173.302 137.922) (width 1.5) (layer F.Cu) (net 11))
 (segment (start 192.532 141.33) (end 194.35 141.33) (width 1.5) (layer F.Cu) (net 11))
 (segment (start 196.3 143.28) (end 196.3 156.72) (width 1.5) (layer F.Cu) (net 11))
 (segment (start 179.88 148.55) (end 173.302 141.972) (width 1.5) (layer F.Cu) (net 11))
 (segment (start 196.3 156.72) (end 194.29 158.73) (width 1.5) (layer F.Cu) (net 11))
 (segment (start 179.88 148.55) (end 179.88 148.56) (width 1.5) (layer F.Cu) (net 11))
 (segment (start 179.88 148.56) (end 180.52 149.2) (width 1.5) (layer F.Cu) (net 11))
 (segment (start 180.52 149.2) (end 180.52 157.08) (width 1.5) (layer F.Cu) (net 11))
 (segment (start 182.17 158.73) (end 194.29 158.73) (width 1.5) (layer F.Cu) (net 11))
 (segment (start 180.52 157.08) (end 182.17 158.73) (width 1.5) (layer F.Cu) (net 11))
 (segment (start 160.02 137.922) (end 157.718 137.922) (width 1.5) (layer F.Cu) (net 12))
 (segment (start 166.624 137.922) (end 168.902 137.922) (width 1.5) (layer F.Cu) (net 12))
 (segment (start 160.274 160.02) (end 160.274 156.21) (width 1.5) (layer F.Cu) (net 12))
 (segment (start 160.274 156.21) (end 163.322 153.162) (width 1.5) (layer F.Cu) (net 12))
 (segment (start 163.322 141.224) (end 160.02 137.922) (width 1.5) (layer F.Cu) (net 12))
 (segment (start 163.322 153.162) (end 163.322 141.224) (width 1.5) (layer F.Cu) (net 12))
 (segment (start 166.624 137.922) (end 163.322 141.224) (width 1.5) (layer F.Cu) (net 12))
 (segment (start 157.718 130.522) (end 159.8 130.522) (width 1.5) (layer F.Cu) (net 14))
 (segment (start 159.8 130.522) (end 161.036 129.286) (width 1.5) (layer F.Cu) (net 14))
 (segment (start 161.036 129.286) (end 161.036 120.396) (width 1.5) (layer F.Cu) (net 14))
 (segment (start 161.036 120.396) (end 159.512 118.872) (width 1.5) (layer F.Cu) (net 14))
 (segment (start 159.512 118.872) (end 150.622 118.872) (width 1.5) (layer F.Cu) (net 14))
 (segment (start 149.098 117.348) (end 149.098 109.22) (width 1.5) (layer F.Cu) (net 14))
 (segment (start 150.622 118.872) (end 149.098 117.348) (width 1.5) (layer F.Cu) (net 14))
 (segment (start 153.318 130.522) (end 153.318 132.94) (width 1.5) (layer F.Cu) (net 13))
 (segment (start 153.318 132.94) (end 152.146 134.112) (width 1.5) (layer F.Cu) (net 13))
 (segment (start 152.146 134.112) (end 141.478 134.112) (width 1.5) (layer F.Cu) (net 13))
 (segment (start 141.478 134.112) (end 140.208 132.842) (width 1.5) (layer F.Cu) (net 13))
 (segment (start 140.208 132.842) (end 140.208 118.364) (width 1.5) (layer F.Cu) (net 13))
 (segment (start 144.018 114.554) (end 144.018 109.22) (width 1.5) (layer F.Cu) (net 13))
 (segment (start 140.208 118.364) (end 144.018 114.554) (width 1.5) (layer F.Cu) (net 13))
 (segment (start 182.372 114.046) (end 182.372 109.22) (width 1.5) (layer F.Cu) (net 15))
 (segment (start 173.302 132.916) (end 174.498 134.112) (width 1.5) (layer F.Cu) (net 15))
 (segment (start 173.302 130.522) (end 173.302 132.916) (width 1.5) (layer F.Cu) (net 15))
 (segment (start 174.498 134.112) (end 186.182 134.112) (width 1.5) (layer F.Cu) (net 15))
 (segment (start 186.182 134.112) (end 187.452 132.842) (width 1.5) (layer F.Cu) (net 15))
 (segment (start 187.452 132.842) (end 187.452 119.126) (width 1.5) (layer F.Cu) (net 15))
 (segment (start 187.452 119.126) (end 182.372 114.046) (width 1.5) (layer F.Cu) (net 15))
 (segment (start 168.902 130.522) (end 167.098 130.522) (width 1.5) (layer F.Cu) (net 16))
 (segment (start 167.098 130.522) (end 165.862 129.286) (width 1.5) (layer F.Cu) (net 16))
 (segment (start 165.862 129.286) (end 165.862 120.142) (width 1.5) (layer F.Cu) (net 16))
 (segment (start 165.862 120.142) (end 167.132 118.872) (width 1.5) (layer F.Cu) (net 16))
 (segment (start 167.132 118.872) (end 175.514 118.872) (width 1.5) (layer F.Cu) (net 16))
 (segment (start 177.292 117.094) (end 177.292 109.22) (width 1.5) (layer F.Cu) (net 16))
 (segment (start 175.514 118.872) (end 177.292 117.094) (width 1.5) (layer F.Cu) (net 16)))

